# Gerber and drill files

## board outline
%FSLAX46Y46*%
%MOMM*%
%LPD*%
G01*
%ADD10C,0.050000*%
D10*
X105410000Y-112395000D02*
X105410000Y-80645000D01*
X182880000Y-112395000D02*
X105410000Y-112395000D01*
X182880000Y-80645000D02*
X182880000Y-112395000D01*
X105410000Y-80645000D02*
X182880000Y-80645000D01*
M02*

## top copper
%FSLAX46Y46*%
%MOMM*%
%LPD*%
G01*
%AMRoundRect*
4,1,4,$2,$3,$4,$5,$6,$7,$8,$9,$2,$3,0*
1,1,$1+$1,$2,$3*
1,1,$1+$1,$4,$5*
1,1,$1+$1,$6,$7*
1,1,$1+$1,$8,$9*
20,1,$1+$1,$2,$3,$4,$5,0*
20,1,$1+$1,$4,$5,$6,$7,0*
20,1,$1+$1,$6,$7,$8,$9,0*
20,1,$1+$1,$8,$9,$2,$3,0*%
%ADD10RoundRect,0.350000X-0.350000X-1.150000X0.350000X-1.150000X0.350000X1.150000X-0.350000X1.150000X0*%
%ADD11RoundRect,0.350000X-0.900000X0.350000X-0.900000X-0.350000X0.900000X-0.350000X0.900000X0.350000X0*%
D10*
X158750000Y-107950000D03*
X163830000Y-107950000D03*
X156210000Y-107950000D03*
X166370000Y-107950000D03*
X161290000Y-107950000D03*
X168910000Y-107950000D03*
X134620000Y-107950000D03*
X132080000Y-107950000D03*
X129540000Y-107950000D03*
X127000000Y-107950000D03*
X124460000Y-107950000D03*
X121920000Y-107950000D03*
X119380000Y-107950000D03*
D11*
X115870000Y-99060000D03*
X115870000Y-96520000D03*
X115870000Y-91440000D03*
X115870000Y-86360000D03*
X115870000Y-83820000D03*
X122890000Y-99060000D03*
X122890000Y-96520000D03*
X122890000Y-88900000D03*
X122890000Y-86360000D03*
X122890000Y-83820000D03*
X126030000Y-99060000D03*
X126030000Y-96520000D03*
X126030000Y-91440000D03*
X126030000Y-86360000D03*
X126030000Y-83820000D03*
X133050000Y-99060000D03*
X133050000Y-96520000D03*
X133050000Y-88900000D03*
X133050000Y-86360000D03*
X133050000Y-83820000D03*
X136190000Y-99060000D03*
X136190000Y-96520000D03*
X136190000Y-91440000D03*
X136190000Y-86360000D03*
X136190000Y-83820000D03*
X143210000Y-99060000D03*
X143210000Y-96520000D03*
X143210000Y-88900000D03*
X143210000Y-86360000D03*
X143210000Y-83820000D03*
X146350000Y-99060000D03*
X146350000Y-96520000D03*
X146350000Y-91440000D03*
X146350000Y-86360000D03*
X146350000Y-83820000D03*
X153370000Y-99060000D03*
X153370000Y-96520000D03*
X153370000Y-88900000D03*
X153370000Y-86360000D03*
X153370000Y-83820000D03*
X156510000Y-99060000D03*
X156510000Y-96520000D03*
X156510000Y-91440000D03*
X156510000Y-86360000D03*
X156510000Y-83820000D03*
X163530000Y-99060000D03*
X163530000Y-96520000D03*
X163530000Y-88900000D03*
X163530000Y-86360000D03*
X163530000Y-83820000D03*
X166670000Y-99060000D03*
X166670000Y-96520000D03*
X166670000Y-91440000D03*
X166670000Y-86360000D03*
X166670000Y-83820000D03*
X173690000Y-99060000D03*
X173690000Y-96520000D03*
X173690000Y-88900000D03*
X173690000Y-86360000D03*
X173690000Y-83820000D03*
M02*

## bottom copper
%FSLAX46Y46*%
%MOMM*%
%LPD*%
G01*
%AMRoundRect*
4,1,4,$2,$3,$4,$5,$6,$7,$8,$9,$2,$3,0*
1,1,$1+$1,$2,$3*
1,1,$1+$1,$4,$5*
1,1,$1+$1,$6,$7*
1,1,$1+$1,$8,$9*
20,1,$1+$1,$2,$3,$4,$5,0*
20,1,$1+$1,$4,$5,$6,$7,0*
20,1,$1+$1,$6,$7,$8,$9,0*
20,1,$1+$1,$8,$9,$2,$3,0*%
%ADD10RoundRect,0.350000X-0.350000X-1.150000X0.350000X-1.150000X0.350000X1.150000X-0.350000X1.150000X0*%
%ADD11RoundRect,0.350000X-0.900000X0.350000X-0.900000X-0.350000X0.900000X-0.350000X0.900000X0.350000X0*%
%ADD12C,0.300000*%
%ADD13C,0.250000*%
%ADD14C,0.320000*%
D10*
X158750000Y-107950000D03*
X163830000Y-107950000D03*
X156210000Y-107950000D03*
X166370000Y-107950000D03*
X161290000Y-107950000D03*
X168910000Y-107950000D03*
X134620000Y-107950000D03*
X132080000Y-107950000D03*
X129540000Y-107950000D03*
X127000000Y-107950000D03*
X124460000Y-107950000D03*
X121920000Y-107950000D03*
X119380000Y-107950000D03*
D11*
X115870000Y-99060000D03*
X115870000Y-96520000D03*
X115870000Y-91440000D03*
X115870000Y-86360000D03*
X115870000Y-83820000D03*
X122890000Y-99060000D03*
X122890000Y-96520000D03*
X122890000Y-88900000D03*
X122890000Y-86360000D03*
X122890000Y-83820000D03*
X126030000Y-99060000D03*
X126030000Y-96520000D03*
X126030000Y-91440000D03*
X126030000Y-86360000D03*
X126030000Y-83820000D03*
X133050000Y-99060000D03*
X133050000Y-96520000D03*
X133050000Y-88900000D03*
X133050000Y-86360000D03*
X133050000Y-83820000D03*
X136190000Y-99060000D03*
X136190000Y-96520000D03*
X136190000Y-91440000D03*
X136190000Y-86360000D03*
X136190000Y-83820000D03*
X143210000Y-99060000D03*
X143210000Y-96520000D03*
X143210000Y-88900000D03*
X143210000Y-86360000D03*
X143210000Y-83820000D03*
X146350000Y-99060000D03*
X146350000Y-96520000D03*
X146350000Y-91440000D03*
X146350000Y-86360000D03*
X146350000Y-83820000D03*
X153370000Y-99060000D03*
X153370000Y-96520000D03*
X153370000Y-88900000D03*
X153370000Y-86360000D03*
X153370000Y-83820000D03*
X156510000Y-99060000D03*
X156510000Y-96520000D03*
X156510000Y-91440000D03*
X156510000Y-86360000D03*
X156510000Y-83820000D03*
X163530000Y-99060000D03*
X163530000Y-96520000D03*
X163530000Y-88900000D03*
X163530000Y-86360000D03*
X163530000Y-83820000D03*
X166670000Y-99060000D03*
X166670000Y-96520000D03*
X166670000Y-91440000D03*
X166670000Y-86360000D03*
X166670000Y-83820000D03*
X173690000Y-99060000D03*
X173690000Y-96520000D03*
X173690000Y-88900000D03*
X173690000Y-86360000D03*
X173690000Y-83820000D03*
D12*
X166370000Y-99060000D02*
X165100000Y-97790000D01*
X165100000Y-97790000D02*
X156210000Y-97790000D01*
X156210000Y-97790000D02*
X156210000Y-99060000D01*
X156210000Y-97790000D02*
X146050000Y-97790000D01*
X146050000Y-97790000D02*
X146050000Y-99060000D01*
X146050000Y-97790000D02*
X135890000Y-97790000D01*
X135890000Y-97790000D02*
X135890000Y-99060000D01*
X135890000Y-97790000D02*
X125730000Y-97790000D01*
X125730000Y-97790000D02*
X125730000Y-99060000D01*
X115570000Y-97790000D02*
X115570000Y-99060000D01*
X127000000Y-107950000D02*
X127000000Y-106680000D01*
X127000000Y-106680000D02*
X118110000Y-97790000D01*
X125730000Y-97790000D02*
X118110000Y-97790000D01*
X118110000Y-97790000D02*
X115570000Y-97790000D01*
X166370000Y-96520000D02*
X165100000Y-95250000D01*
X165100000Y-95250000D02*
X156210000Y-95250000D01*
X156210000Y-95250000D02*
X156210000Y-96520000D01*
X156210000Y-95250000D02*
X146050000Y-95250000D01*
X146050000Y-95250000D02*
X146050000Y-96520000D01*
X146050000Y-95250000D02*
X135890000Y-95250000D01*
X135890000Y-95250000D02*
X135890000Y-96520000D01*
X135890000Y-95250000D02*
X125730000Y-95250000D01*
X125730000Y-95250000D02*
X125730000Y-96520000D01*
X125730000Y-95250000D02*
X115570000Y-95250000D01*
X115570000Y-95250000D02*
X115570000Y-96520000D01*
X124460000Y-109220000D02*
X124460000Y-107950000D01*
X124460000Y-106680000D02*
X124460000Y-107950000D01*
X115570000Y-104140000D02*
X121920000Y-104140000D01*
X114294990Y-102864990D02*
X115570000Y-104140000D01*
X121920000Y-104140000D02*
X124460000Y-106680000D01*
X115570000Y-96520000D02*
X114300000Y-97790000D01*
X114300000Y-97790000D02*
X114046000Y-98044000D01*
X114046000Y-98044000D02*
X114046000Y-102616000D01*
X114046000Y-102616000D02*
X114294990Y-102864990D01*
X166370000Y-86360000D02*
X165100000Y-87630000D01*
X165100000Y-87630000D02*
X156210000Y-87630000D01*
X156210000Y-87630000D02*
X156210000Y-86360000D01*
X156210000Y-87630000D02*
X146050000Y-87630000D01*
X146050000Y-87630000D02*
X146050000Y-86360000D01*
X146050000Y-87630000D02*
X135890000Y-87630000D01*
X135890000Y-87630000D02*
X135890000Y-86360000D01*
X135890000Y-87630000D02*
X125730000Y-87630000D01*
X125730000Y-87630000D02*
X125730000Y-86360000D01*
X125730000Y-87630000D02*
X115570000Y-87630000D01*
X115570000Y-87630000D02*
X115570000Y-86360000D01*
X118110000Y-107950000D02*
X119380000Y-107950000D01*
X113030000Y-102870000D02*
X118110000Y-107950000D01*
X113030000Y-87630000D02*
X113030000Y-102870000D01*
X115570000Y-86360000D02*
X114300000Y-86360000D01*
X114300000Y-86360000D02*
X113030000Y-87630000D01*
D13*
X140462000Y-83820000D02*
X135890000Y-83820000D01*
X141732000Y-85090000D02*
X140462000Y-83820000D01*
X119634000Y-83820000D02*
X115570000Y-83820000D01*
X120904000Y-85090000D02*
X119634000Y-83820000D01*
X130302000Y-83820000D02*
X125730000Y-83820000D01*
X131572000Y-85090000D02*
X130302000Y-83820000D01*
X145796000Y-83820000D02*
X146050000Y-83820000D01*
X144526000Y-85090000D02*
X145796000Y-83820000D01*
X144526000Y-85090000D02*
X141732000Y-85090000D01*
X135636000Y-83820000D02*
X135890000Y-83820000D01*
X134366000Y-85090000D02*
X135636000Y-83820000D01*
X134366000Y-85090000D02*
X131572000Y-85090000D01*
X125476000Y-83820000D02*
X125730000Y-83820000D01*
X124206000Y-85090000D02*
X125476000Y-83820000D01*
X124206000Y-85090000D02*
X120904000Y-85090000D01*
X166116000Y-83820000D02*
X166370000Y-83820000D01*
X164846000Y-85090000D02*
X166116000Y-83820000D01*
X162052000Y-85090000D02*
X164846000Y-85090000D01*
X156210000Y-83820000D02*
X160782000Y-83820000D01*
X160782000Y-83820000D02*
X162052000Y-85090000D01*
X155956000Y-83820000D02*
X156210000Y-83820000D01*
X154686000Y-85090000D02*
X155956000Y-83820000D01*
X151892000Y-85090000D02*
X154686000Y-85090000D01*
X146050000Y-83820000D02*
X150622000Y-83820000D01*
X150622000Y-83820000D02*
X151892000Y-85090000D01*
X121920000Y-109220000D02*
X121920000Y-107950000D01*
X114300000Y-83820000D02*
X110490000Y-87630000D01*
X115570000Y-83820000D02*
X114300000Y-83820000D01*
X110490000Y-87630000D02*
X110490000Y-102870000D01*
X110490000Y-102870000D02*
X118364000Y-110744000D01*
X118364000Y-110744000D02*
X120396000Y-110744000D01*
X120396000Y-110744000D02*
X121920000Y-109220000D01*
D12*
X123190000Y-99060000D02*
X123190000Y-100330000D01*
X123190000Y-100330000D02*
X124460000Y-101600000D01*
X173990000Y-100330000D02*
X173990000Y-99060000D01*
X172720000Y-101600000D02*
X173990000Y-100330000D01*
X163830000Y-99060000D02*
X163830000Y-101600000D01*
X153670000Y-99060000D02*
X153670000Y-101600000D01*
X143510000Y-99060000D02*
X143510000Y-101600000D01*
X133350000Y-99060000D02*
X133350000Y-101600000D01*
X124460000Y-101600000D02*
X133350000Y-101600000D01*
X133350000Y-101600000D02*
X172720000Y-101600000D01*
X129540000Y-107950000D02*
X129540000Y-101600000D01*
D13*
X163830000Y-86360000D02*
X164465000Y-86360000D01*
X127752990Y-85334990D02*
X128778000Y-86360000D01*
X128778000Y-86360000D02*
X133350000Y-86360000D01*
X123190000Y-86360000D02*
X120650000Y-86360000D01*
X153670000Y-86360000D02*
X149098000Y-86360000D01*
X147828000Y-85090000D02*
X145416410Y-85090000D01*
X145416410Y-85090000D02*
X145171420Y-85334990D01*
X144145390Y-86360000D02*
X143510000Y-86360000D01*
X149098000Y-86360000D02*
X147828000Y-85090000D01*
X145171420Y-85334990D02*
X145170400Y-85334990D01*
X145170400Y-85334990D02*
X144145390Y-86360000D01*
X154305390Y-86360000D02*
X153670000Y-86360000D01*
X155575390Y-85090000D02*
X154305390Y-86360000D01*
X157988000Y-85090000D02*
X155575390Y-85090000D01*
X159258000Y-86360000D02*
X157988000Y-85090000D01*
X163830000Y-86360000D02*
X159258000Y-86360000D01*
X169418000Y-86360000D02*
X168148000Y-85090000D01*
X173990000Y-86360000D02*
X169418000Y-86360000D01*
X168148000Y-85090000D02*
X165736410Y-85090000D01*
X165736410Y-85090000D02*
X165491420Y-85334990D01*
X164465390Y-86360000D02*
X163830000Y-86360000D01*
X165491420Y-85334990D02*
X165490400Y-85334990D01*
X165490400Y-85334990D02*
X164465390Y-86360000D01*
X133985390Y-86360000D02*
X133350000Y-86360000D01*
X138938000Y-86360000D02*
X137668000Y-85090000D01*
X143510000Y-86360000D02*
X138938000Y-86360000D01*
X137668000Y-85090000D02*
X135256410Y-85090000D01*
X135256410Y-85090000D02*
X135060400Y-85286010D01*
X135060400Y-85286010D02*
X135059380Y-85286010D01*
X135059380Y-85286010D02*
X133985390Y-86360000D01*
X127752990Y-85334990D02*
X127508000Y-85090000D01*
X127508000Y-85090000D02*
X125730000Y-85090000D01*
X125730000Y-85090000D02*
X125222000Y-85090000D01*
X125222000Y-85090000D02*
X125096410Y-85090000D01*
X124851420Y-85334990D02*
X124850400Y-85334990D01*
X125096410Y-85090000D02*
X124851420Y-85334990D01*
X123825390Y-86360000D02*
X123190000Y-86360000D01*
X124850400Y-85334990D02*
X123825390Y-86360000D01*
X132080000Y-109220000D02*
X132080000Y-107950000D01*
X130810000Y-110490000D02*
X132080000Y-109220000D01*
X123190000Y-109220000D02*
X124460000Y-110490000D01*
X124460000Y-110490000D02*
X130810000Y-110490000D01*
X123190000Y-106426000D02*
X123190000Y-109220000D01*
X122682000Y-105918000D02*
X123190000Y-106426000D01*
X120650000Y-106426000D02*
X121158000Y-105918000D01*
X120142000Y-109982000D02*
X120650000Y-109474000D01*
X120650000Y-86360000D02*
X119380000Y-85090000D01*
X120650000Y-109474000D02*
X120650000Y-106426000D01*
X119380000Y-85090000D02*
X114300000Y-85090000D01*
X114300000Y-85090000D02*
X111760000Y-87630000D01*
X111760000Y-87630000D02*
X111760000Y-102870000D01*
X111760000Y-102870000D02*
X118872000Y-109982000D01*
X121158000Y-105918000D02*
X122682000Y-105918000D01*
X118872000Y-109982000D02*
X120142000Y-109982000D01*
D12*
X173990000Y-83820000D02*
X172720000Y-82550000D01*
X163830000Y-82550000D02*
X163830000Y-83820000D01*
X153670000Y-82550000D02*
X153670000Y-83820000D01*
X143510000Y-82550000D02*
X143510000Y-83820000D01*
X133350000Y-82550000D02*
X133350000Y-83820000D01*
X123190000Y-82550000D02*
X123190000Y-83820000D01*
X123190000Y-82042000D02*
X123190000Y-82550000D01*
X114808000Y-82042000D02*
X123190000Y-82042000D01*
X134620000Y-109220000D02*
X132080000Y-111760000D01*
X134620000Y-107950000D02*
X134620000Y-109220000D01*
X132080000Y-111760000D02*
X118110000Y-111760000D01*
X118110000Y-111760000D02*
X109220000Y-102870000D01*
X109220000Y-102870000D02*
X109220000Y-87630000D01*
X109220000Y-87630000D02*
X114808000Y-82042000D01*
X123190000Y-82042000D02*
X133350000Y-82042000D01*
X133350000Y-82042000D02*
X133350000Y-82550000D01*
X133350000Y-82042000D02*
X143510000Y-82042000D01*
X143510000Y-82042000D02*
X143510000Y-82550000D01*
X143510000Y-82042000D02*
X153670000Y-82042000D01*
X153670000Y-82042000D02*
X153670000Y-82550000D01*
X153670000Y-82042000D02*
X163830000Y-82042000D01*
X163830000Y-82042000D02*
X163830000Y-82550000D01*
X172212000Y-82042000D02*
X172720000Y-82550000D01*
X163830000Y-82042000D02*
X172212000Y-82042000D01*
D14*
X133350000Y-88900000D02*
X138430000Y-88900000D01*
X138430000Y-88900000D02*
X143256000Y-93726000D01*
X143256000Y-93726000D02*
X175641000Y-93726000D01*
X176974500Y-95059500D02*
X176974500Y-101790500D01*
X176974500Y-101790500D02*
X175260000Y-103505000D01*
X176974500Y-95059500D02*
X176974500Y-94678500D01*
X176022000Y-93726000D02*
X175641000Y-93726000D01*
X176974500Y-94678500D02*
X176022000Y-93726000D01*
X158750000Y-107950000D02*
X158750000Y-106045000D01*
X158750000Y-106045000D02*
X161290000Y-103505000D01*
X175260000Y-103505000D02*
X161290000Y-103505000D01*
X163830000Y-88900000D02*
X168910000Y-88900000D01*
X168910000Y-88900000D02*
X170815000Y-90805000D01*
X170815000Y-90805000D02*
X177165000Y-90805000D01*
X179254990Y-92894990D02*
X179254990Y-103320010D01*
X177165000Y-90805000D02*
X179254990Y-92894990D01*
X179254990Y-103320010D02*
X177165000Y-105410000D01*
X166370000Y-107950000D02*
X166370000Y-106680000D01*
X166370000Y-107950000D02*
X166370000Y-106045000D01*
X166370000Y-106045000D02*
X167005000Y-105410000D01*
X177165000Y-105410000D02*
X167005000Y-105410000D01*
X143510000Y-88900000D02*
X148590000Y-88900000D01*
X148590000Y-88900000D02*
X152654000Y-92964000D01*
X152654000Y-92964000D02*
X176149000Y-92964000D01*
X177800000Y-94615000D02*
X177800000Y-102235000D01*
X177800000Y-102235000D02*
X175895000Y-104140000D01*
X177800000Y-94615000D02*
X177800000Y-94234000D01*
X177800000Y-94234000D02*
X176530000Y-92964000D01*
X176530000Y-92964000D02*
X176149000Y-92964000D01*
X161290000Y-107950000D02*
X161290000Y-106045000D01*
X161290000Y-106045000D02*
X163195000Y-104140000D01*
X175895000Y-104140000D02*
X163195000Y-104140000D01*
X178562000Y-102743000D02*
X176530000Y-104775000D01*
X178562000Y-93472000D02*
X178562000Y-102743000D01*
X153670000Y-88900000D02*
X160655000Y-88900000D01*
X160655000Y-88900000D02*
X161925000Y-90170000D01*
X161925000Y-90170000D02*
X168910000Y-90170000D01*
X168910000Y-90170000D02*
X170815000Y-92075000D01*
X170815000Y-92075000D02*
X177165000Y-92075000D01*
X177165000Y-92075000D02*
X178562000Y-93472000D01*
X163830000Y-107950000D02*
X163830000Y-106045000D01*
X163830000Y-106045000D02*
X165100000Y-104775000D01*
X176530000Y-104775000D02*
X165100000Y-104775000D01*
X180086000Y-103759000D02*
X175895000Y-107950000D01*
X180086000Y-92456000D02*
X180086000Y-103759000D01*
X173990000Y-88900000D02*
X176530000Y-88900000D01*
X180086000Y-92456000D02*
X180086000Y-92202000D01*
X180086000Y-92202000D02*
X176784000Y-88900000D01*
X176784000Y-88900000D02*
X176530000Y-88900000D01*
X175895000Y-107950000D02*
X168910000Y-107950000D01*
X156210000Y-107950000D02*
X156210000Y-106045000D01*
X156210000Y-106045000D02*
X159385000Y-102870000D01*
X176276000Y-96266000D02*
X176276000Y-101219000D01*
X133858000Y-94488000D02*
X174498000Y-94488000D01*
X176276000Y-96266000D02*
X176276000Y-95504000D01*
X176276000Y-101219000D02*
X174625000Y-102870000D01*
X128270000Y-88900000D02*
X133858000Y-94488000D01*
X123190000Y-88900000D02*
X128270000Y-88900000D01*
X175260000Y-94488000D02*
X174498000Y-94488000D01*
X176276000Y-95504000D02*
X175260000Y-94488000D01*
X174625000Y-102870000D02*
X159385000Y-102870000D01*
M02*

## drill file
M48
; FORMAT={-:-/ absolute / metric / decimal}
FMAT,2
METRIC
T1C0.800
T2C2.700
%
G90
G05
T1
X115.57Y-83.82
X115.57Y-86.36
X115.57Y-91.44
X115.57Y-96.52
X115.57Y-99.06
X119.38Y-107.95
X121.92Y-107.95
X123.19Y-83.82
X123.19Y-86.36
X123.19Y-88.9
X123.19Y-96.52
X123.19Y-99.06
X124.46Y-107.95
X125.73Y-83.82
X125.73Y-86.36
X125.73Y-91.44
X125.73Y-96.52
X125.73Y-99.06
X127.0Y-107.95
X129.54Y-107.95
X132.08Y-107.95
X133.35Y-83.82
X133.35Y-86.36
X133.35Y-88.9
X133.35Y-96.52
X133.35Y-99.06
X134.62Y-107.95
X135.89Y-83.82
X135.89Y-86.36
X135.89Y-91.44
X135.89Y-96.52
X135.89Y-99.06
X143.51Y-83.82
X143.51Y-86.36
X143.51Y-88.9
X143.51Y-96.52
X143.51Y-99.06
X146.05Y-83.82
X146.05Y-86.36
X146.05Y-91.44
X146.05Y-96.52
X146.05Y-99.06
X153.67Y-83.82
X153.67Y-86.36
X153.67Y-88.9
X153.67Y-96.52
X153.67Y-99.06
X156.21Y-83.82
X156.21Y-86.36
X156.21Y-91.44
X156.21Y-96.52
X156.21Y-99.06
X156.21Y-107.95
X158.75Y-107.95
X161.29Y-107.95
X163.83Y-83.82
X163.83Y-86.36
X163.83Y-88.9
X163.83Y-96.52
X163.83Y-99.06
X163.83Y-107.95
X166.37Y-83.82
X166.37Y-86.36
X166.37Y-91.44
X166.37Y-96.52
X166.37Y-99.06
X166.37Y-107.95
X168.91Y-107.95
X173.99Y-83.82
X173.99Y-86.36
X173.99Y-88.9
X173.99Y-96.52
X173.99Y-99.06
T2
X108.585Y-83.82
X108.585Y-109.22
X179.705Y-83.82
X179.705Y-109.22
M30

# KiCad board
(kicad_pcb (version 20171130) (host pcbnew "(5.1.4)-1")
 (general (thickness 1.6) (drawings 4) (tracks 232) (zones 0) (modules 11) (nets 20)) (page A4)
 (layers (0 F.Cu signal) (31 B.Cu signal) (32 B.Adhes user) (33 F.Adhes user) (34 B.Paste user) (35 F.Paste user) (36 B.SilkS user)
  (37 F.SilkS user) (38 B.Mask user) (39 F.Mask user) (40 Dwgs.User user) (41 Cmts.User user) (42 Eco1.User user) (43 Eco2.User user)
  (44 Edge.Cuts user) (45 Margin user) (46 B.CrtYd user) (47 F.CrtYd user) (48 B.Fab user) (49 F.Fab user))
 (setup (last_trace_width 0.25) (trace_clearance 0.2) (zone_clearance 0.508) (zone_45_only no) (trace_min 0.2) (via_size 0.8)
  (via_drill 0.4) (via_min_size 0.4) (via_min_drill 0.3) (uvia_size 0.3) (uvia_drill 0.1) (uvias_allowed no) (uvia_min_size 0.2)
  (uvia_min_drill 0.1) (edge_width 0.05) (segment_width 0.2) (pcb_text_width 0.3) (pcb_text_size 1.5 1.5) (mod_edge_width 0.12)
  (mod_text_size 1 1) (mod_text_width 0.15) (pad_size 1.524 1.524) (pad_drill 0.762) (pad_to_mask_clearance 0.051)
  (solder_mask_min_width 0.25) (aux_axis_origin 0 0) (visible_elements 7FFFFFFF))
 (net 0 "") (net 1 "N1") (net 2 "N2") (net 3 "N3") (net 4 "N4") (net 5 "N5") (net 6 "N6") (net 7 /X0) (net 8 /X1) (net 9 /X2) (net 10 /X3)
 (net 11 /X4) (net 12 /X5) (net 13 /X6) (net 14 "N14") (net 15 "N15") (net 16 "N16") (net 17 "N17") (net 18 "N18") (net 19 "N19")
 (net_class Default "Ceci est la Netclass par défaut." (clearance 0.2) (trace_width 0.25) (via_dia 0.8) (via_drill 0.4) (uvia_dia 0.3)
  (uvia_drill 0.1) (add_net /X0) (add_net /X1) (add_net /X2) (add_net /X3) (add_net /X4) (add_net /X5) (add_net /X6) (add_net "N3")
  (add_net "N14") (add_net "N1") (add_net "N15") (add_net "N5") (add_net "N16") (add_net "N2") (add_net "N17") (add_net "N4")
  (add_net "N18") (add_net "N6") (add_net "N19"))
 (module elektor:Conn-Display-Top (layer F.Cu) (at 127 111.76)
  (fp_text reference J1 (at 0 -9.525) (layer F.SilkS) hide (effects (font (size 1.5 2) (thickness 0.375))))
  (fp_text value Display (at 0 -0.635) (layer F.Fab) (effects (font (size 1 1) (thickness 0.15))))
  (pad 2 thru_hole roundrect (at 31.75 -3.81) (size 1.4 3) (drill 0.8) (layers *.Cu *.Mask) (roundrect_rratio 0.25) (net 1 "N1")
   (zone_connect 0))
  (pad 4 thru_hole roundrect (at 36.83 -3.81) (size 1.4 3) (drill 0.8) (layers *.Cu *.Mask) (roundrect_rratio 0.25) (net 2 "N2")
   (zone_connect 0))
  (pad 1 thru_hole roundrect (at 29.21 -3.81) (size 1.4 3) (drill 0.8) (layers *.Cu *.Mask) (roundrect_rratio 0.25) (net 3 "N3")
   (zone_connect 0))
  (pad 5 thru_hole roundrect (at 39.37 -3.81) (size 1.4 3) (drill 0.8) (layers *.Cu *.Mask) (roundrect_rratio 0.25) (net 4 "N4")
   (zone_connect 0))
  (pad 3 thru_hole roundrect (at 34.29 -3.81) (size 1.4 3) (drill 0.8) (layers *.Cu *.Mask) (roundrect_rratio 0.25) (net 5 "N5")
   (zone_connect 0))
  (pad 6 thru_hole roundrect (at 41.91 -3.81) (size 1.4 3) (drill 0.8) (layers *.Cu *.Mask) (roundrect_rratio 0.25) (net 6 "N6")
   (zone_connect 0))
  (pad a thru_hole roundrect (at 7.62 -3.81) (size 1.4 3) (drill 0.8) (layers *.Cu *.Mask) (roundrect_rratio 0.25) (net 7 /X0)
   (zone_connect 0))
  (pad b thru_hole roundrect (at 5.08 -3.81) (size 1.4 3) (drill 0.8) (layers *.Cu *.Mask) (roundrect_rratio 0.25) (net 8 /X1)
   (zone_connect 0))
  (pad c thru_hole roundrect (at 2.54 -3.81) (size 1.4 3) (drill 0.8) (layers *.Cu *.Mask) (roundrect_rratio 0.25) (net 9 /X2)
   (zone_connect 0))
  (pad d thru_hole roundrect (at 0 -3.81) (size 1.4 3) (drill 0.8) (layers *.Cu *.Mask) (roundrect_rratio 0.25) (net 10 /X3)
   (zone_connect 0))
  (pad e thru_hole roundrect (at -2.54 -3.81) (size 1.4 3) (drill 0.8) (layers *.Cu *.Mask) (roundrect_rratio 0.25) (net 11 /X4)
   (zone_connect 0))
  (pad f thru_hole roundrect (at -5.08 -3.81) (size 1.4 3) (drill 0.8) (layers *.Cu *.Mask) (roundrect_rratio 0.25) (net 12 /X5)
   (zone_connect 0))
  (pad g thru_hole roundrect (at -7.62 -3.81) (size 1.4 3) (drill 0.8) (layers *.Cu *.Mask) (roundrect_rratio 0.25) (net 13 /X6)
   (zone_connect 0)))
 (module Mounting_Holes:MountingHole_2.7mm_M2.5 (layer F.Cu) (at 108.585 83.82)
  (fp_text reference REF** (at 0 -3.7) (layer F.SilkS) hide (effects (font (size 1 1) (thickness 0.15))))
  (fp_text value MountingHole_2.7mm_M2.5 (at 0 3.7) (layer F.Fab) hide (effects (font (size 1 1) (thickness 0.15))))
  (pad 1 np_thru_hole circle (at 0 0) (size 2.7 2.7) (drill 2.7) (layers *.Cu *.Mask)))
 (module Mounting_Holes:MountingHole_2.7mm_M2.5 (layer F.Cu) (at 108.585 109.22)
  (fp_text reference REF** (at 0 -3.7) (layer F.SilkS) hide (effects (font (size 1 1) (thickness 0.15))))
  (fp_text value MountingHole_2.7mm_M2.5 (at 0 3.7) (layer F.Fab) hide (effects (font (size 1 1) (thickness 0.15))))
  (pad 1 np_thru_hole circle (at 0 0) (size 2.7 2.7) (drill 2.7) (layers *.Cu *.Mask)))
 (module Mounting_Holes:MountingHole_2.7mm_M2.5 (layer F.Cu) (at 179.705 109.22)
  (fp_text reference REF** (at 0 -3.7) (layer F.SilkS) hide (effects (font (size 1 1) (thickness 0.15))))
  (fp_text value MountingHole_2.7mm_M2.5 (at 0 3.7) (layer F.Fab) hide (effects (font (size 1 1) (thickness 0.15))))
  (pad 1 np_thru_hole circle (at 0 0) (size 2.7 2.7) (drill 2.7) (layers *.Cu *.Mask)))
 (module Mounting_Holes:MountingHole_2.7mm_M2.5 (layer F.Cu) (at 179.705 83.82)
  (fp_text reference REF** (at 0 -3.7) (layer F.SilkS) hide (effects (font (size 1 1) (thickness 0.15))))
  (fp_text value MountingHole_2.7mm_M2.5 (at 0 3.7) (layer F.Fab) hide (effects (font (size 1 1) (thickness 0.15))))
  (pad 1 np_thru_hole circle (at 0 0) (size 2.7 2.7) (drill 2.7) (layers *.Cu *.Mask)))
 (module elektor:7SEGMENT (layer F.Cu) (at 119.38 87.63)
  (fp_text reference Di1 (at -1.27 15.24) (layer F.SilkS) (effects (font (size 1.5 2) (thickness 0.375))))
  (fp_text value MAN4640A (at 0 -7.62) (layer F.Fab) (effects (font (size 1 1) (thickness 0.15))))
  (pad 7 thru_hole roundrect (at -3.81 11.43 270) (size 1.4 2.5) (drill 0.8 (offset 0 -0.3)) (layers *.Cu *.Mask) (roundrect_rratio 0.25)
   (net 10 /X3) (zone_connect 0))
  (pad 6 thru_hole roundrect (at -3.81 8.89 270) (size 1.4 2.5) (drill 0.8 (offset 0 -0.3)) (layers *.Cu *.Mask) (roundrect_rratio 0.25)
   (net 11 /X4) (zone_connect 0))
  (pad 4 thru_hole roundrect (at -3.81 3.81 270) (size 1.4 2.5) (drill 0.8 (offset 0 -0.3)) (layers *.Cu *.Mask) (roundrect_rratio 0.25)
   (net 3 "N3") (zone_connect 0))
  (pad 2 thru_hole roundrect (at -3.81 -1.27 270) (size 1.4 2.5) (drill 0.8 (offset 0 -0.3)) (layers *.Cu *.Mask) (roundrect_rratio 0.25)
   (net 13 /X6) (zone_connect 0))
  (pad 1 thru_hole roundrect (at -3.81 -3.81 270) (size 1.4 2.5) (drill 0.8 (offset 0 -0.3)) (layers *.Cu *.Mask) (roundrect_rratio 0.25)
   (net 12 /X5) (zone_connect 0))
  (pad 8 thru_hole roundrect (at 3.81 11.43 270) (size 1.4 2.5) (drill 0.8 (offset 0 0.3)) (layers *.Cu *.Mask) (roundrect_rratio 0.25)
   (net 9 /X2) (zone_connect 0))
  (pad 9 thru_hole roundrect (at 3.81 8.89 270) (size 1.4 2.5) (drill 0.8 (offset 0 0.3)) (layers *.Cu *.Mask) (roundrect_rratio 0.25)
   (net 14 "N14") (zone_connect 0))
  (pad 12 thru_hole roundrect (at 3.81 1.27 270) (size 1.4 2.5) (drill 0.8 (offset 0 0.3)) (layers *.Cu *.Mask) (roundrect_rratio 0.25)
   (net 3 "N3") (zone_connect 0))
  (pad 13 thru_hole roundrect (at 3.81 -1.27 270) (size 1.4 2.5) (drill 0.8 (offset 0 0.3)) (layers *.Cu *.Mask) (roundrect_rratio 0.25)
   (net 8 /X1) (zone_connect 0))
  (pad 14 thru_hole roundrect (at 3.81 -3.81 270) (size 1.4 2.5) (drill 0.8 (offset 0 0.3)) (layers *.Cu *.Mask) (roundrect_rratio 0.25)
   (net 7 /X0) (zone_connect 0)))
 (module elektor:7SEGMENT (layer F.Cu) (at 129.54 87.63)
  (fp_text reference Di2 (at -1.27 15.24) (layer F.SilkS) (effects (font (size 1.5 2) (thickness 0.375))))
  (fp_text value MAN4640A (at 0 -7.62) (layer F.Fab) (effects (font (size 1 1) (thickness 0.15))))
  (pad 7 thru_hole roundrect (at -3.81 11.43 270) (size 1.4 2.5) (drill 0.8 (offset 0 -0.3)) (layers *.Cu *.Mask) (roundrect_rratio 0.25)
   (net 10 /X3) (zone_connect 0))
  (pad 6 thru_hole roundrect (at -3.81 8.89 270) (size 1.4 2.5) (drill 0.8 (offset 0 -0.3)) (layers *.Cu *.Mask) (roundrect_rratio 0.25)
   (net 11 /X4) (zone_connect 0))
  (pad 4 thru_hole roundrect (at -3.81 3.81 270) (size 1.4 2.5) (drill 0.8 (offset 0 -0.3)) (layers *.Cu *.Mask) (roundrect_rratio 0.25)
   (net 1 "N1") (zone_connect 0))
  (pad 2 thru_hole roundrect (at -3.81 -1.27 270) (size 1.4 2.5) (drill 0.8 (offset 0 -0.3)) (layers *.Cu *.Mask) (roundrect_rratio 0.25)
   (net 13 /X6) (zone_connect 0))
  (pad 1 thru_hole roundrect (at -3.81 -3.81 270) (size 1.4 2.5) (drill 0.8 (offset 0 -0.3)) (layers *.Cu *.Mask) (roundrect_rratio 0.25)
   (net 12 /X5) (zone_connect 0))
  (pad 8 thru_hole roundrect (at 3.81 11.43 270) (size 1.4 2.5) (drill 0.8 (offset 0 0.3)) (layers *.Cu *.Mask) (roundrect_rratio 0.25)
   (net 9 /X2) (zone_connect 0))
  (pad 9 thru_hole roundrect (at 3.81 8.89 270) (size 1.4 2.5) (drill 0.8 (offset 0 0.3)) (layers *.Cu *.Mask) (roundrect_rratio 0.25)
   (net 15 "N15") (zone_connect 0))
  (pad 12 thru_hole roundrect (at 3.81 1.27 270) (size 1.4 2.5) (drill 0.8 (offset 0 0.3)) (layers *.Cu *.Mask) (roundrect_rratio 0.25)
   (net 1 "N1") (zone_connect 0))
  (pad 13 thru_hole roundrect (at 3.81 -1.27 270) (size 1.4 2.5) (drill 0.8 (offset 0 0.3)) (layers *.Cu *.Mask) (roundrect_rratio 0.25)
   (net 8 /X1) (zone_connect 0))
  (pad 14 thru_hole roundrect (at 3.81 -3.81 270) (size 1.4 2.5) (drill 0.8 (offset 0 0.3)) (layers *.Cu *.Mask) (roundrect_rratio 0.25)
   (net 7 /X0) (zone_connect 0)))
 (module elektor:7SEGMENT (layer F.Cu) (at 139.7 87.63)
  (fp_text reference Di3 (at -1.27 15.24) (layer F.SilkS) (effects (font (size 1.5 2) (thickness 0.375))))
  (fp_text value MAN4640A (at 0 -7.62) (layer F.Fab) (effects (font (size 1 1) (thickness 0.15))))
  (pad 7 thru_hole roundrect (at -3.81 11.43 270) (size 1.4 2.5) (drill 0.8 (offset 0 -0.3)) (layers *.Cu *.Mask) (roundrect_rratio 0.25)
   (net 10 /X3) (zone_connect 0))
  (pad 6 thru_hole roundrect (at -3.81 8.89 270) (size 1.4 2.5) (drill 0.8 (offset 0 -0.3)) (layers *.Cu *.Mask) (roundrect_rratio 0.25)
   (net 11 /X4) (zone_connect 0))
  (pad 4 thru_hole roundrect (at -3.81 3.81 270) (size 1.4 2.5) (drill 0.8 (offset 0 -0.3)) (layers *.Cu *.Mask) (roundrect_rratio 0.25)
   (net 5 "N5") (zone_connect 0))
  (pad 2 thru_hole roundrect (at -3.81 -1.27 270) (size 1.4 2.5) (drill 0.8 (offset 0 -0.3)) (layers *.Cu *.Mask) (roundrect_rratio 0.25)
   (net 13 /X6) (zone_connect 0))
  (pad 1 thru_hole roundrect (at -3.81 -3.81 270) (size 1.4 2.5) (drill 0.8 (offset 0 -0.3)) (layers *.Cu *.Mask) (roundrect_rratio 0.25)
   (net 12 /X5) (zone_connect 0))
  (pad 8 thru_hole roundrect (at 3.81 11.43 270) (size 1.4 2.5) (drill 0.8 (offset 0 0.3)) (layers *.Cu *.Mask) (roundrect_rratio 0.25)
   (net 9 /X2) (zone_connect 0))
  (pad 9 thru_hole roundrect (at 3.81 8.89 270) (size 1.4 2.5) (drill 0.8 (offset 0 0.3)) (layers *.Cu *.Mask) (roundrect_rratio 0.25)
   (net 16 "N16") (zone_connect 0))
  (pad 12 thru_hole roundrect (at 3.81 1.27 270) (size 1.4 2.5) (drill 0.8 (offset 0 0.3)) (layers *.Cu *.Mask) (roundrect_rratio 0.25)
   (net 5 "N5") (zone_connect 0))
  (pad 13 thru_hole roundrect (at 3.81 -1.27 270) (size 1.4 2.5) (drill 0.8 (offset 0 0.3)) (layers *.Cu *.Mask) (roundrect_rratio 0.25)
   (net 8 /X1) (zone_connect 0))
  (pad 14 thru_hole roundrect (at 3.81 -3.81 270) (size 1.4 2.5) (drill 0.8 (offset 0 0.3)) (layers *.Cu *.Mask) (roundrect_rratio 0.25)
   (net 7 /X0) (zone_connect 0)))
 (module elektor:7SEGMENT (layer F.Cu) (at 149.86 87.63)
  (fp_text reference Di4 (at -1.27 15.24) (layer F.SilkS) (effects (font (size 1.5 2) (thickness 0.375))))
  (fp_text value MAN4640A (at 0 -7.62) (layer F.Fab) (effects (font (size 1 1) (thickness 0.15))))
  (pad 7 thru_hole roundrect (at -3.81 11.43 270) (size 1.4 2.5) (drill 0.8 (offset 0 -0.3)) (layers *.Cu *.Mask) (roundrect_rratio 0.25)
   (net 10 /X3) (zone_connect 0))
  (pad 6 thru_hole roundrect (at -3.81 8.89 270) (size 1.4 2.5) (drill 0.8 (offset 0 -0.3)) (layers *.Cu *.Mask) (roundrect_rratio 0.25)
   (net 11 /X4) (zone_connect 0))
  (pad 4 thru_hole roundrect (at -3.81 3.81 270) (size 1.4 2.5) (drill 0.8 (offset 0 -0.3)) (layers *.Cu *.Mask) (roundrect_rratio 0.25)
   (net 2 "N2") (zone_connect 0))
  (pad 2 thru_hole roundrect (at -3.81 -1.27 270) (size 1.4 2.5) (drill 0.8 (offset 0 -0.3)) (layers *.Cu *.Mask) (roundrect_rratio 0.25)
   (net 13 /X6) (zone_connect 0))
  (pad 1 thru_hole roundrect (at -3.81 -3.81 270) (size 1.4 2.5) (drill 0.8 (offset 0 -0.3)) (layers *.Cu *.Mask) (roundrect_rratio 0.25)
   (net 12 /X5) (zone_connect 0))
  (pad 8 thru_hole roundrect (at 3.81 11.43 270) (size 1.4 2.5) (drill 0.8 (offset 0 0.3)) (layers *.Cu *.Mask) (roundrect_rratio 0.25)
   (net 9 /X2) (zone_connect 0))
  (pad 9 thru_hole roundrect (at 3.81 8.89 270) (size 1.4 2.5) (drill 0.8 (offset 0 0.3)) (layers *.Cu *.Mask) (roundrect_rratio 0.25)
   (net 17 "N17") (zone_connect 0))
  (pad 12 thru_hole roundrect (at 3.81 1.27 270) (size 1.4 2.5) (drill 0.8 (offset 0 0.3)) (layers *.Cu *.Mask) (roundrect_rratio 0.25)
   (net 2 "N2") (zone_connect 0))
  (pad 13 thru_hole roundrect (at 3.81 -1.27 270) (size 1.4 2.5) (drill 0.8 (offset 0 0.3)) (layers *.Cu *.Mask) (roundrect_rratio 0.25)
   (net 8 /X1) (zone_connect 0))
  (pad 14 thru_hole roundrect (at 3.81 -3.81 270) (size 1.4 2.5) (drill 0.8 (offset 0 0.3)) (layers *.Cu *.Mask) (roundrect_rratio 0.25)
   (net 7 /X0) (zone_connect 0)))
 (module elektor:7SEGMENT (layer F.Cu) (at 160.02 87.63)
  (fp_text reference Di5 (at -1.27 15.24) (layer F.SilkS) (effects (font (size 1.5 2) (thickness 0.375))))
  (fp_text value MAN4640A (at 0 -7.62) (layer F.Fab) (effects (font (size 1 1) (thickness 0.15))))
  (pad 7 thru_hole roundrect (at -3.81 11.43 270) (size 1.4 2.5) (drill 0.8 (offset 0 -0.3)) (layers *.Cu *.Mask) (roundrect_rratio 0.25)
   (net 10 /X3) (zone_connect 0))
  (pad 6 thru_hole roundrect (at -3.81 8.89 270) (size 1.4 2.5) (drill 0.8 (offset 0 -0.3)) (layers *.Cu *.Mask) (roundrect_rratio 0.25)
   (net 11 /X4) (zone_connect 0))
  (pad 4 thru_hole roundrect (at -3.81 3.81 270) (size 1.4 2.5) (drill 0.8 (offset 0 -0.3)) (layers *.Cu *.Mask) (roundrect_rratio 0.25)
   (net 4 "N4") (zone_connect 0))
  (pad 2 thru_hole roundrect (at -3.81 -1.27 270) (size 1.4 2.5) (drill 0.8 (offset 0 -0.3)) (layers *.Cu *.Mask) (roundrect_rratio 0.25)
   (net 13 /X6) (zone_connect 0))
  (pad 1 thru_hole roundrect (at -3.81 -3.81 270) (size 1.4 2.5) (drill 0.8 (offset 0 -0.3)) (layers *.Cu *.Mask) (roundrect_rratio 0.25)
   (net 12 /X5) (zone_connect 0))
  (pad 8 thru_hole roundrect (at 3.81 11.43 270) (size 1.4 2.5) (drill 0.8 (offset 0 0.3)) (layers *.Cu *.Mask) (roundrect_rratio 0.25)
   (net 9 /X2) (zone_connect 0))
  (pad 9 thru_hole roundrect (at 3.81 8.89 270) (size 1.4 2.5) (drill 0.8 (offset 0 0.3)) (layers *.Cu *.Mask) (roundrect_rratio 0.25)
   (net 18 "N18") (zone_connect 0))
  (pad 12 thru_hole roundrect (at 3.81 1.27 270) (size 1.4 2.5) (drill 0.8 (offset 0 0.3)) (layers *.Cu *.Mask) (roundrect_rratio 0.25)
   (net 4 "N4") (zone_connect 0))
  (pad 13 thru_hole roundrect (at 3.81 -1.27 270) (size 1.4 2.5) (drill 0.8 (offset 0 0.3)) (layers *.Cu *.Mask) (roundrect_rratio 0.25)
   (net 8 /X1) (zone_connect 0))
  (pad 14 thru_hole roundrect (at 3.81 -3.81 270) (size 1.4 2.5) (drill 0.8 (offset 0 0.3)) (layers *.Cu *.Mask) (roundrect_rratio 0.25)
   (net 7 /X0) (zone_connect 0)))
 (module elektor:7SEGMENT (layer F.Cu) (at 170.18 87.63)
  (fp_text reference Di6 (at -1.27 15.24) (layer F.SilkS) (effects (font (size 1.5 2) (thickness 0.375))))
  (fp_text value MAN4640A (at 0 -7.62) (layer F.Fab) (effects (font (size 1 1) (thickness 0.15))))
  (pad 7 thru_hole roundrect (at -3.81 11.43 270) (size 1.4 2.5) (drill 0.8 (offset 0 -0.3)) (layers *.Cu *.Mask) (roundrect_rratio 0.25)
   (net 10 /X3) (zone_connect 0))
  (pad 6 thru_hole roundrect (at -3.81 8.89 270) (size 1.4 2.5) (drill 0.8 (offset 0 -0.3)) (layers *.Cu *.Mask) (roundrect_rratio 0.25)
   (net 11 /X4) (zone_connect 0))
  (pad 4 thru_hole roundrect (at -3.81 3.81 270) (size 1.4 2.5) (drill 0.8 (offset 0 -0.3)) (layers *.Cu *.Mask) (roundrect_rratio 0.25)
   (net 6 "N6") (zone_connect 0))
  (pad 2 thru_hole roundrect (at -3.81 -1.27 270) (size 1.4 2.5) (drill 0.8 (offset 0 -0.3)) (layers *.Cu *.Mask) (roundrect_rratio 0.25)
   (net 13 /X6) (zone_connect 0))
  (pad 1 thru_hole roundrect (at -3.81 -3.81 270) (size 1.4 2.5) (drill 0.8 (offset 0 -0.3)) (layers *.Cu *.Mask) (roundrect_rratio 0.25)
   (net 12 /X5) (zone_connect 0))
  (pad 8 thru_hole roundrect (at 3.81 11.43 270) (size 1.4 2.5) (drill 0.8 (offset 0 0.3)) (layers *.Cu *.Mask) (roundrect_rratio 0.25)
   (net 9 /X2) (zone_connect 0))
  (pad 9 thru_hole roundrect (at 3.81 8.89 270) (size 1.4 2.5) (drill 0.8 (offset 0 0.3)) (layers *.Cu *.Mask) (roundrect_rratio 0.25)
   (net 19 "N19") (zone_connect 0))
  (pad 12 thru_hole roundrect (at 3.81 1.27 270) (size 1.4 2.5) (drill 0.8 (offset 0 0.3)) (layers *.Cu *.Mask) (roundrect_rratio 0.25)
   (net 6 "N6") (zone_connect 0))
  (pad 13 thru_hole roundrect (at 3.81 -1.27 270) (size 1.4 2.5) (drill 0.8 (offset 0 0.3)) (layers *.Cu *.Mask) (roundrect_rratio 0.25)
   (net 8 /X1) (zone_connect 0))
  (pad 14 thru_hole roundrect (at 3.81 -3.81 270) (size 1.4 2.5) (drill 0.8 (offset 0 0.3)) (layers *.Cu *.Mask) (roundrect_rratio 0.25)
   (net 7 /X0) (zone_connect 0)))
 (gr_line (start 105.41 112.395) (end 105.41 80.645) (layer Edge.Cuts) (width 0.05))
 (gr_line (start 182.88 112.395) (end 105.41 112.395) (layer Edge.Cuts) (width 0.05))
 (gr_line (start 182.88 80.645) (end 182.88 112.395) (layer Edge.Cuts) (width 0.05))
 (gr_line (start 105.41 80.645) (end 182.88 80.645) (layer Edge.Cuts) (width 0.05))
 (segment (start 166.37 99.06) (end 165.1 97.79) (width 0.3) (layer B.Cu) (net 10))
 (segment (start 165.1 97.79) (end 156.21 97.79) (width 0.3) (layer B.Cu) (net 10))
 (segment (start 156.21 97.79) (end 156.21 99.06) (width 0.3) (layer B.Cu) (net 10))
 (segment (start 156.21 97.79) (end 146.05 97.79) (width 0.3) (layer B.Cu) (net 10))
 (segment (start 146.05 97.79) (end 146.05 99.06) (width 0.3) (layer B.Cu) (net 10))
 (segment (start 146.05 97.79) (end 135.89 97.79) (width 0.3) (layer B.Cu) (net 10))
 (segment (start 135.89 97.79) (end 135.89 99.06) (width 0.3) (layer B.Cu) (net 10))
 (segment (start 135.89 97.79) (end 125.73 97.79) (width 0.3) (layer B.Cu) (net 10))
 (segment (start 125.73 97.79) (end 125.73 99.06) (width 0.3) (layer B.Cu) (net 10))
 (segment (start 115.57 97.79) (end 115.57 99.06) (width 0.3) (layer B.Cu) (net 10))
 (segment (start 127 107.95) (end 127 106.68) (width 0.3) (layer B.Cu) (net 10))
 (segment (start 127 106.68) (end 118.11 97.79) (width 0.3) (layer B.Cu) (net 10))
 (segment (start 125.73 97.79) (end 118.11 97.79) (width 0.3) (layer B.Cu) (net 10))
 (segment (start 118.11 97.79) (end 115.57 97.79) (width 0.3) (layer B.Cu) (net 10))
 (segment (start 166.37 96.52) (end 165.1 95.25) (width 0.3) (layer B.Cu) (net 11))
 (segment (start 165.1 95.25) (end 156.21 95.25) (width 0.3) (layer B.Cu) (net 11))
 (segment (start 156.21 95.25) (end 156.21 96.52) (width 0.3) (layer B.Cu) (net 11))
 (segment (start 156.21 95.25) (end 146.05 95.25) (width 0.3) (layer B.Cu) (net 11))
 (segment (start 146.05 95.25) (end 146.05 96.52) (width 0.3) (layer B.Cu) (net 11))
 (segment (start 146.05 95.25) (end 135.89 95.25) (width 0.3) (layer B.Cu) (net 11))
 (segment (start 135.89 95.25) (end 135.89 96.52) (width 0.3) (layer B.Cu) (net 11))
 (segment (start 135.89 95.25) (end 125.73 95.25) (width 0.3) (layer B.Cu) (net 11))
 (segment (start 125.73 95.25) (end 125.73 96.52) (width 0.3) (layer B.Cu) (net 11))
 (segment (start 125.73 95.25) (end 115.57 95.25) (width 0.3) (layer B.Cu) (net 11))
 (segment (start 115.57 95.25) (end 115.57 96.52) (width 0.3) (layer B.Cu) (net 11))
 (segment (start 124.46 109.22) (end 124.46 107.95) (width 0.3) (layer B.Cu) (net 11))
 (segment (start 124.46 106.68) (end 124.46 107.95) (width 0.3) (layer B.Cu) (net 11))
 (segment (start 115.57 104.14) (end 121.92 104.14) (width 0.3) (layer B.Cu) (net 11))
 (segment (start 114.29499 102.86499) (end 115.57 104.14) (width 0.3) (layer B.Cu) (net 11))
 (segment (start 121.92 104.14) (end 124.46 106.68) (width 0.3) (layer B.Cu) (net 11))
 (segment (start 115.57 96.52) (end 114.3 97.79) (width 0.3) (layer B.Cu) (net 11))
 (segment (start 114.3 97.79) (end 114.046 98.044) (width 0.3) (layer B.Cu) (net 11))
 (segment (start 114.046 98.044) (end 114.046 102.616) (width 0.3) (layer B.Cu) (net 11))
 (segment (start 114.046 102.616) (end 114.29499 102.86499) (width 0.3) (layer B.Cu) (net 11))
 (segment (start 166.37 86.36) (end 165.1 87.63) (width 0.3) (layer B.Cu) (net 13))
 (segment (start 165.1 87.63) (end 156.21 87.63) (width 0.3) (layer B.Cu) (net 13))
 (segment (start 156.21 87.63) (end 156.21 86.36) (width 0.3) (layer B.Cu) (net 13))
 (segment (start 156.21 87.63) (end 146.05 87.63) (width 0.3) (layer B.Cu) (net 13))
 (segment (start 146.05 87.63) (end 146.05 86.36) (width 0.3) (layer B.Cu) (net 13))
 (segment (start 146.05 87.63) (end 135.89 87.63) (width 0.3) (layer B.Cu) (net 13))
 (segment (start 135.89 87.63) (end 135.89 86.36) (width 0.3) (layer B.Cu) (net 13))
 (segment (start 135.89 87.63) (end 125.73 87.63) (width 0.3) (layer B.Cu) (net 13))
 (segment (start 125.73 87.63) (end 125.73 86.36) (width 0.3) (layer B.Cu) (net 13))
 (segment (start 125.73 87.63) (end 115.57 87.63) (width 0.3) (layer B.Cu) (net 13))
 (segment (start 115.57 87.63) (end 115.57 86.36) (width 0.3) (layer B.Cu) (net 13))
 (segment (start 118.11 107.95) (end 119.38 107.95) (width 0.3) (layer B.Cu) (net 13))
 (segment (start 113.03 102.87) (end 118.11 107.95) (width 0.3) (layer B.Cu) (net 13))
 (segment (start 113.03 87.63) (end 113.03 102.87) (width 0.3) (layer B.Cu) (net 13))
 (segment (start 115.57 86.36) (end 114.3 86.36) (width 0.3) (layer B.Cu) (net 13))
 (segment (start 114.3 86.36) (end 113.03 87.63) (width 0.3) (layer B.Cu) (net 13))
 (segment (start 140.462 83.82) (end 135.89 83.82) (width 0.25) (layer B.Cu) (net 12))
 (segment (start 141.732 85.09) (end 140.462 83.82) (width 0.25) (layer B.Cu) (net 12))
 (segment (start 119.634 83.82) (end 115.57 83.82) (width 0.25) (layer B.Cu) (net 12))
 (segment (start 120.904 85.09) (end 119.634 83.82) (width 0.25) (layer B.Cu) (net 12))
 (segment (start 130.302 83.82) (end 125.73 83.82) (width 0.25) (layer B.Cu) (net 12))
 (segment (start 131.572 85.09) (end 130.302 83.82) (width 0.25) (layer B.Cu) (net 12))
 (segment (start 145.796 83.82) (end 146.05 83.82) (width 0.25) (layer B.Cu) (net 12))
 (segment (start 144.526 85.09) (end 145.796 83.82) (width 0.25) (layer B.Cu) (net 12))
 (segment (start 144.526 85.09) (end 141.732 85.09) (width 0.25) (layer B.Cu) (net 12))
 (segment (start 135.636 83.82) (end 135.89 83.82) (width 0.25) (layer B.Cu) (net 12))
 (segment (start 134.366 85.09) (end 135.636 83.82) (width 0.25) (layer B.Cu) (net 12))
 (segment (start 134.366 85.09) (end 131.572 85.09) (width 0.25) (layer B.Cu) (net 12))
 (segment (start 125.476 83.82) (end 125.73 83.82) (width 0.25) (layer B.Cu) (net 12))
 (segment (start 124.206 85.09) (end 125.476 83.82) (width 0.25) (layer B.Cu) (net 12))
 (segment (start 124.206 85.09) (end 120.904 85.09) (width 0.25) (layer B.Cu) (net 12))
 (segment (start 166.116 83.82) (end 166.37 83.82) (width 0.25) (layer B.Cu) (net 12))
 (segment (start 164.846 85.09) (end 166.116 83.82) (width 0.25) (layer B.Cu) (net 12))
 (segment (start 162.052 85.09) (end 164.846 85.09) (width 0.25) (layer B.Cu) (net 12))
 (segment (start 156.21 83.82) (end 160.782 83.82) (width 0.25) (layer B.Cu) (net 12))
 (segment (start 160.782 83.82) (end 162.052 85.09) (width 0.25) (layer B.Cu) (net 12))
 (segment (start 155.956 83.82) (end 156.21 83.82) (width 0.25) (layer B.Cu) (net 12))
 (segment (start 154.686 85.09) (end 155.956 83.82) (width 0.25) (layer B.Cu) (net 12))
 (segment (start 151.892 85.09) (end 154.686 85.09) (width 0.25) (layer B.Cu) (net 12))
 (segment (start 146.05 83.82) (end 150.622 83.82) (width 0.25) (layer B.Cu) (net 12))
 (segment (start 150.622 83.82) (end 151.892 85.09) (width 0.25) (layer B.Cu) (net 12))
 (segment (start 121.92 109.22) (end 121.92 107.95) (width 0.25) (layer B.Cu) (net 12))
 (segment (start 114.3 83.82) (end 110.49 87.63) (width 0.25) (layer B.Cu) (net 12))
 (segment (start 115.57 83.82) (end 114.3 83.82) (width 0.25) (layer B.Cu) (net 12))
 (segment (start 110.49 87.63) (end 110.49 102.87) (width 0.25) (layer B.Cu) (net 12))
 (segment (start 110.49 102.87) (end 118.364 110.744) (width 0.25) (layer B.Cu) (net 12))
 (segment (start 118.364 110.744) (end 120.396 110.744) (width 0.25) (layer B.Cu) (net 12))
 (segment (start 120.396 110.744) (end 121.92 109.22) (width 0.25) (layer B.Cu) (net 12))
 (segment (start 123.19 99.06) (end 123.19 100.33) (width 0.3) (layer B.Cu) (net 9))
 (segment (start 123.19 100.33) (end 124.46 101.6) (width 0.3) (layer B.Cu) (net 9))
 (segment (start 173.99 100.33) (end 173.99 99.06) (width 0.3) (layer B.Cu) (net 9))
 (segment (start 172.72 101.6) (end 173.99 100.33) (width 0.3) (layer B.Cu) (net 9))
 (segment (start 163.83 99.06) (end 163.83 101.6) (width 0.3) (layer B.Cu) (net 9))
 (segment (start 153.67 99.06) (end 153.67 101.6) (width 0.3) (layer B.Cu) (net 9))
 (segment (start 143.51 99.06) (end 143.51 101.6) (width 0.3) (layer B.Cu) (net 9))
 (segment (start 133.35 99.06) (end 133.35 101.6) (width 0.3) (layer B.Cu) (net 9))
 (segment (start 124.46 101.6) (end 133.35 101.6) (width 0.3) (layer B.Cu) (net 9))
 (segment (start 133.35 101.6) (end 172.72 101.6) (width 0.3) (layer B.Cu) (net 9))
 (segment (start 129.54 107.95) (end 129.54 101.6) (width 0.3) (layer B.Cu) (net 9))
 (segment (start 163.83 86.36) (end 164.465 86.36) (width 0.25) (layer B.Cu) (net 8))
 (segment (start 127.75299 85.33499) (end 128.778 86.36) (width 0.25) (layer B.Cu) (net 8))
 (segment (start 128.778 86.36) (end 133.35 86.36) (width 0.25) (layer B.Cu) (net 8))
 (segment (start 123.19 86.36) (end 120.65 86.36) (width 0.25) (layer B.Cu) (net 8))
 (segment (start 153.67 86.36) (end 149.098 86.36) (width 0.25) (layer B.Cu) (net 8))
 (segment (start 147.828 85.09) (end 145.41641 85.09) (width 0.25) (layer B.Cu) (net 8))
 (segment (start 145.41641 85.09) (end 145.17142 85.33499) (width 0.25) (layer B.Cu) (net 8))
 (segment (start 144.14539 86.36) (end 143.51 86.36) (width 0.25) (layer B.Cu) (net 8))
 (segment (start 149.098 86.36) (end 147.828 85.09) (width 0.25) (layer B.Cu) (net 8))
 (segment (start 145.17142 85.33499) (end 145.1704 85.33499) (width 0.25) (layer B.Cu) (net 8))
 (segment (start 145.1704 85.33499) (end 144.14539 86.36) (width 0.25) (layer B.Cu) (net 8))
 (segment (start 154.30539 86.36) (end 153.67 86.36) (width 0.25) (layer B.Cu) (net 8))
 (segment (start 155.57539 85.09) (end 154.30539 86.36) (width 0.25) (layer B.Cu) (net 8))
 (segment (start 157.988 85.09) (end 155.57539 85.09) (width 0.25) (layer B.Cu) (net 8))
 (segment (start 159.258 86.36) (end 157.988 85.09) (width 0.25) (layer B.Cu) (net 8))
 (segment (start 163.83 86.36) (end 159.258 86.36) (width 0.25) (layer B.Cu) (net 8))
 (segment (start 169.418 86.36) (end 168.148 85.09) (width 0.25) (layer B.Cu) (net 8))
 (segment (start 173.99 86.36) (end 169.418 86.36) (width 0.25) (layer B.Cu) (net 8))
 (segment (start 168.148 85.09) (end 165.73641 85.09) (width 0.25) (layer B.Cu) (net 8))
 (segment (start 165.73641 85.09) (end 165.49142 85.33499) (width 0.25) (layer B.Cu) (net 8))
 (segment (start 164.46539 86.36) (end 163.83 86.36) (width 0.25) (layer B.Cu) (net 8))
 (segment (start 165.49142 85.33499) (end 165.4904 85.33499) (width 0.25) (layer B.Cu) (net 8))
 (segment (start 165.4904 85.33499) (end 164.46539 86.36) (width 0.25) (layer B.Cu) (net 8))
 (segment (start 133.98539 86.36) (end 133.35 86.36) (width 0.25) (layer B.Cu) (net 8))
 (segment (start 138.938 86.36) (end 137.668 85.09) (width 0.25) (layer B.Cu) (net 8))
 (segment (start 143.51 86.36) (end 138.938 86.36) (width 0.25) (layer B.Cu) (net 8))
 (segment (start 137.668 85.09) (end 135.25641 85.09) (width 0.25) (layer B.Cu) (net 8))
 (segment (start 135.25641 85.09) (end 135.0604 85.28601) (width 0.25) (layer B.Cu) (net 8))
 (segment (start 135.0604 85.28601) (end 135.05938 85.28601) (width 0.25) (layer B.Cu) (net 8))
 (segment (start 135.05938 85.28601) (end 133.98539 86.36) (width 0.25) (layer B.Cu) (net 8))
 (segment (start 127.75299 85.33499) (end 127.508 85.09) (width 0.25) (layer B.Cu) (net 8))
 (segment (start 127.508 85.09) (end 125.73 85.09) (width 0.25) (layer B.Cu) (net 8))
 (segment (start 125.73 85.09) (end 125.222 85.09) (width 0.25) (layer B.Cu) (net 8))
 (segment (start 125.222 85.09) (end 125.09641 85.09) (width 0.25) (layer B.Cu) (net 8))
 (segment (start 124.85142 85.33499) (end 124.8504 85.33499) (width 0.25) (layer B.Cu) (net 8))
 (segment (start 125.09641 85.09) (end 124.85142 85.33499) (width 0.25) (layer B.Cu) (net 8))
 (segment (start 123.82539 86.36) (end 123.19 86.36) (width 0.25) (layer B.Cu) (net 8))
 (segment (start 124.8504 85.33499) (end 123.82539 86.36) (width 0.25) (layer B.Cu) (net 8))
 (segment (start 132.08 109.22) (end 132.08 107.95) (width 0.25) (layer B.Cu) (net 8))
 (segment (start 130.81 110.49) (end 132.08 109.22) (width 0.25) (layer B.Cu) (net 8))
 (segment (start 123.19 109.22) (end 124.46 110.49) (width 0.25) (layer B.Cu) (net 8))
 (segment (start 124.46 110.49) (end 130.81 110.49) (width 0.25) (layer B.Cu) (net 8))
 (segment (start 123.19 106.426) (end 123.19 109.22) (width 0.25) (layer B.Cu) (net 8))
 (segment (start 122.682 105.918) (end 123.19 106.426) (width 0.25) (layer B.Cu) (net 8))
 (segment (start 120.65 106.426) (end 121.158 105.918) (width 0.25) (layer B.Cu) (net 8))
 (segment (start 120.142 109.982) (end 120.65 109.474) (width 0.25) (layer B.Cu) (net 8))
 (segment (start 120.65 86.36) (end 119.38 85.09) (width 0.25) (layer B.Cu) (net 8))
 (segment (start 120.65 109.474) (end 120.65 106.426) (width 0.25) (layer B.Cu) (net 8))
 (segment (start 119.38 85.09) (end 114.3 85.09) (width 0.25) (layer B.Cu) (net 8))
 (segment (start 114.3 85.09) (end 111.76 87.63) (width 0.25) (layer B.Cu) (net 8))
 (segment (start 111.76 87.63) (end 111.76 102.87) (width 0.25) (layer B.Cu) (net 8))
 (segment (start 111.76 102.87) (end 118.872 109.982) (width 0.25) (layer B.Cu) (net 8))
 (segment (start 121.158 105.918) (end 122.682 105.918) (width 0.25) (layer B.Cu) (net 8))
 (segment (start 118.872 109.982) (end 120.142 109.982) (width 0.25) (layer B.Cu) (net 8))
 (segment (start 173.99 83.82) (end 172.72 82.55) (width 0.3) (layer B.Cu) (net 7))
 (segment (start 163.83 82.55) (end 163.83 83.82) (width 0.3) (layer B.Cu) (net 7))
 (segment (start 153.67 82.55) (end 153.67 83.82) (width 0.3) (layer B.Cu) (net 7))
 (segment (start 143.51 82.55) (end 143.51 83.82) (width 0.3) (layer B.Cu) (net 7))
 (segment (start 133.35 82.55) (end 133.35 83.82) (width 0.3) (layer B.Cu) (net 7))
 (segment (start 123.19 82.55) (end 123.19 83.82) (width 0.3) (layer B.Cu) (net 7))
 (segment (start 123.19 82.042) (end 123.19 82.55) (width 0.3) (layer B.Cu) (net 7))
 (segment (start 114.808 82.042) (end 123.19 82.042) (width 0.3) (layer B.Cu) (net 7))
 (segment (start 134.62 109.22) (end 132.08 111.76) (width 0.3) (layer B.Cu) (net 7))
 (segment (start 134.62 107.95) (end 134.62 109.22) (width 0.3) (layer B.Cu) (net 7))
 (segment (start 132.08 111.76) (end 118.11 111.76) (width 0.3) (layer B.Cu) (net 7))
 (segment (start 118.11 111.76) (end 109.22 102.87) (width 0.3) (layer B.Cu) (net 7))
 (segment (start 109.22 102.87) (end 109.22 87.63) (width 0.3) (layer B.Cu) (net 7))
 (segment (start 109.22 87.63) (end 114.808 82.042) (width 0.3) (layer B.Cu) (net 7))
 (segment (start 123.19 82.042) (end 133.35 82.042) (width 0.3) (layer B.Cu) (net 7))
 (segment (start 133.35 82.042) (end 133.35 82.55) (width 0.3) (layer B.Cu) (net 7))
 (segment (start 133.35 82.042) (end 143.51 82.042) (width 0.3) (layer B.Cu) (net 7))
 (segment (start 143.51 82.042) (end 143.51 82.55) (width 0.3) (layer B.Cu) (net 7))
 (segment (start 143.51 82.042) (end 153.67 82.042) (width 0.3) (layer B.Cu) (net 7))
 (segment (start 153.67 82.042) (end 153.67 82.55) (width 0.3) (layer B.Cu) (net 7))
 (segment (start 153.67 82.042) (end 163.83 82.042) (width 0.3) (layer B.Cu) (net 7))
 (segment (start 163.83 82.042) (end 163.83 82.55) (width 0.3) (layer B.Cu) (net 7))
 (segment (start 172.212 82.042) (end 172.72 82.55) (width 0.3) (layer B.Cu) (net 7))
 (segment (start 163.83 82.042) (end 172.212 82.042) (width 0.3) (layer B.Cu) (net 7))
 (segment (start 133.35 88.9) (end 138.43 88.9) (width 0.32) (layer B.Cu) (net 1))
 (segment (start 138.43 88.9) (end 143.256 93.726) (width 0.32) (layer B.Cu) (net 1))
 (segment (start 143.256 93.726) (end 175.641 93.726) (width 0.32) (layer B.Cu) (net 1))
 (segment (start 176.9745 95.0595) (end 176.9745 101.7905) (width 0.32) (layer B.Cu) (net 1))
 (segment (start 176.9745 101.7905) (end 175.26 103.505) (width 0.32) (layer B.Cu) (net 1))
 (segment (start 176.9745 95.0595) (end 176.9745 94.6785) (width 0.32) (layer B.Cu) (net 1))
 (segment (start 176.022 93.726) (end 175.641 93.726) (width 0.32) (layer B.Cu) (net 1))
 (segment (start 176.9745 94.6785) (end 176.022 93.726) (width 0.32) (layer B.Cu) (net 1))
 (segment (start 158.75 107.95) (end 158.75 106.045) (width 0.32) (layer B.Cu) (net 1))
 (segment (start 158.75 106.045) (end 161.29 103.505) (width 0.32) (layer B.Cu) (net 1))
 (segment (start 175.26 103.505) (end 161.29 103.505) (width 0.32) (layer B.Cu) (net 1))
 (segment (start 163.83 88.9) (end 168.91 88.9) (width 0.32) (layer B.Cu) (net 4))
 (segment (start 168.91 88.9) (end 170.815 90.805) (width 0.32) (layer B.Cu) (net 4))
 (segment (start 170.815 90.805) (end 177.165 90.805) (width 0.32) (layer B.Cu) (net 4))
 (segment (start 179.25499 92.89499) (end 179.25499 103.32001) (width 0.32) (layer B.Cu) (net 4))
 (segment (start 177.165 90.805) (end 179.25499 92.89499) (width 0.32) (layer B.Cu) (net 4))
 (segment (start 179.25499 103.32001) (end 177.165 105.41) (width 0.32) (layer B.Cu) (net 4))
 (segment (start 166.37 107.95) (end 166.37 106.68) (width 0.32) (layer B.Cu) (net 4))
 (segment (start 166.37 107.95) (end 166.37 106.045) (width 0.32) (layer B.Cu) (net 4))
 (segment (start 166.37 106.045) (end 167.005 105.41) (width 0.32) (layer B.Cu) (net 4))
 (segment (start 177.165 105.41) (end 167.005 105.41) (width 0.32) (layer B.Cu) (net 4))
 (segment (start 143.51 88.9) (end 148.59 88.9) (width 0.32) (layer B.Cu) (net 5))
 (segment (start 148.59 88.9) (end 152.654 92.964) (width 0.32) (layer B.Cu) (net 5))
 (segment (start 152.654 92.964) (end 176.149 92.964) (width 0.32) (layer B.Cu) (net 5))
 (segment (start 177.8 94.615) (end 177.8 102.235) (width 0.32) (layer B.Cu) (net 5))
 (segment (start 177.8 102.235) (end 175.895 104.14) (width 0.32) (layer B.Cu) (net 5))
 (segment (start 177.8 94.615) (end 177.8 94.234) (width 0.32) (layer B.Cu) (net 5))
 (segment (start 177.8 94.234) (end 176.53 92.964) (width 0.32) (layer B.Cu) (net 5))
 (segment (start 176.53 92.964) (end 176.149 92.964) (width 0.32) (layer B.Cu) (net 5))
 (segment (start 161.29 107.95) (end 161.29 106.045) (width 0.32) (layer B.Cu) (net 5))
 (segment (start 161.29 106.045) (end 163.195 104.14) (width 0.32) (layer B.Cu) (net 5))
 (segment (start 175.895 104.14) (end 163.195 104.14) (width 0.32) (layer B.Cu) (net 5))
 (segment (start 178.562 102.743) (end 176.53 104.775) (width 0.32) (layer B.Cu) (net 2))
 (segment (start 178.562 93.472) (end 178.562 102.743) (width 0.32) (layer B.Cu) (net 2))
 (segment (start 153.67 88.9) (end 160.655 88.9) (width 0.32) (layer B.Cu) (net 2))
 (segment (start 160.655 88.9) (end 161.925 90.17) (width 0.32) (layer B.Cu) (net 2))
 (segment (start 161.925 90.17) (end 168.91 90.17) (width 0.32) (layer B.Cu) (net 2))
 (segment (start 168.91 90.17) (end 170.815 92.075) (width 0.32) (layer B.Cu) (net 2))
 (segment (start 170.815 92.075) (end 177.165 92.075) (width 0.32) (layer B.Cu) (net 2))
 (segment (start 177.165 92.075) (end 178.562 93.472) (width 0.32) (layer B.Cu) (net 2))
 (segment (start 163.83 107.95) (end 163.83 106.045) (width 0.32) (layer B.Cu) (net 2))
 (segment (start 163.83 106.045) (end 165.1 104.775) (width 0.32) (layer B.Cu) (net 2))
 (segment (start 176.53 104.775) (end 165.1 104.775) (width 0.32) (layer B.Cu) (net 2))
 (segment (start 180.086 103.759) (end 175.895 107.95) (width 0.32) (layer B.Cu) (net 6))
 (segment (start 180.086 92.456) (end 180.086 103.759) (width 0.32) (layer B.Cu) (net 6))
 (segment (start 173.99 88.9) (end 176.53 88.9) (width 0.32) (layer B.Cu) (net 6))
 (segment (start 180.086 92.456) (end 180.086 92.202) (width 0.32) (layer B.Cu) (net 6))
 (segment (start 180.086 92.202) (end 176.784 88.9) (width 0.32) (layer B.Cu) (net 6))
 (segment (start 176.784 88.9) (end 176.53 88.9) (width 0.32) (layer B.Cu) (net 6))
 (segment (start 175.895 107.95) (end 168.91 107.95) (width 0.32) (layer B.Cu) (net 6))
 (segment (start 156.21 107.95) (end 156.21 106.045) (width 0.32) (layer B.Cu) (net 3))
 (segment (start 156.21 106.045) (end 159.385 102.87) (width 0.32) (layer B.Cu) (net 3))
 (segment (start 176.276 96.266) (end 176.276 101.219) (width 0.32) (layer B.Cu) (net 3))
 (segment (start 133.858 94.488) (end 174.498 94.488) (width 0.32) (layer B.Cu) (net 3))
 (segment (start 176.276 96.266) (end 176.276 95.504) (width 0.32) (layer B.Cu) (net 3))
 (segment (start 176.276 101.219) (end 174.625 102.87) (width 0.32) (layer B.Cu) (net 3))
 (segment (start 128.27 88.9) (end 133.858 94.488) (width 0.32) (layer B.Cu) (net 3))
 (segment (start 123.19 88.9) (end 128.27 88.9) (width 0.32) (layer B.Cu) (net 3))
 (segment (start 175.26 94.488) (end 174.498 94.488) (width 0.32) (layer B.Cu) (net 3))
 (segment (start 176.276 95.504) (end 175.26 94.488) (width 0.32) (layer B.Cu) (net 3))
 (segment (start 174.625 102.87) (end 159.385 102.87) (width 0.32) (layer B.Cu) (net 3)))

